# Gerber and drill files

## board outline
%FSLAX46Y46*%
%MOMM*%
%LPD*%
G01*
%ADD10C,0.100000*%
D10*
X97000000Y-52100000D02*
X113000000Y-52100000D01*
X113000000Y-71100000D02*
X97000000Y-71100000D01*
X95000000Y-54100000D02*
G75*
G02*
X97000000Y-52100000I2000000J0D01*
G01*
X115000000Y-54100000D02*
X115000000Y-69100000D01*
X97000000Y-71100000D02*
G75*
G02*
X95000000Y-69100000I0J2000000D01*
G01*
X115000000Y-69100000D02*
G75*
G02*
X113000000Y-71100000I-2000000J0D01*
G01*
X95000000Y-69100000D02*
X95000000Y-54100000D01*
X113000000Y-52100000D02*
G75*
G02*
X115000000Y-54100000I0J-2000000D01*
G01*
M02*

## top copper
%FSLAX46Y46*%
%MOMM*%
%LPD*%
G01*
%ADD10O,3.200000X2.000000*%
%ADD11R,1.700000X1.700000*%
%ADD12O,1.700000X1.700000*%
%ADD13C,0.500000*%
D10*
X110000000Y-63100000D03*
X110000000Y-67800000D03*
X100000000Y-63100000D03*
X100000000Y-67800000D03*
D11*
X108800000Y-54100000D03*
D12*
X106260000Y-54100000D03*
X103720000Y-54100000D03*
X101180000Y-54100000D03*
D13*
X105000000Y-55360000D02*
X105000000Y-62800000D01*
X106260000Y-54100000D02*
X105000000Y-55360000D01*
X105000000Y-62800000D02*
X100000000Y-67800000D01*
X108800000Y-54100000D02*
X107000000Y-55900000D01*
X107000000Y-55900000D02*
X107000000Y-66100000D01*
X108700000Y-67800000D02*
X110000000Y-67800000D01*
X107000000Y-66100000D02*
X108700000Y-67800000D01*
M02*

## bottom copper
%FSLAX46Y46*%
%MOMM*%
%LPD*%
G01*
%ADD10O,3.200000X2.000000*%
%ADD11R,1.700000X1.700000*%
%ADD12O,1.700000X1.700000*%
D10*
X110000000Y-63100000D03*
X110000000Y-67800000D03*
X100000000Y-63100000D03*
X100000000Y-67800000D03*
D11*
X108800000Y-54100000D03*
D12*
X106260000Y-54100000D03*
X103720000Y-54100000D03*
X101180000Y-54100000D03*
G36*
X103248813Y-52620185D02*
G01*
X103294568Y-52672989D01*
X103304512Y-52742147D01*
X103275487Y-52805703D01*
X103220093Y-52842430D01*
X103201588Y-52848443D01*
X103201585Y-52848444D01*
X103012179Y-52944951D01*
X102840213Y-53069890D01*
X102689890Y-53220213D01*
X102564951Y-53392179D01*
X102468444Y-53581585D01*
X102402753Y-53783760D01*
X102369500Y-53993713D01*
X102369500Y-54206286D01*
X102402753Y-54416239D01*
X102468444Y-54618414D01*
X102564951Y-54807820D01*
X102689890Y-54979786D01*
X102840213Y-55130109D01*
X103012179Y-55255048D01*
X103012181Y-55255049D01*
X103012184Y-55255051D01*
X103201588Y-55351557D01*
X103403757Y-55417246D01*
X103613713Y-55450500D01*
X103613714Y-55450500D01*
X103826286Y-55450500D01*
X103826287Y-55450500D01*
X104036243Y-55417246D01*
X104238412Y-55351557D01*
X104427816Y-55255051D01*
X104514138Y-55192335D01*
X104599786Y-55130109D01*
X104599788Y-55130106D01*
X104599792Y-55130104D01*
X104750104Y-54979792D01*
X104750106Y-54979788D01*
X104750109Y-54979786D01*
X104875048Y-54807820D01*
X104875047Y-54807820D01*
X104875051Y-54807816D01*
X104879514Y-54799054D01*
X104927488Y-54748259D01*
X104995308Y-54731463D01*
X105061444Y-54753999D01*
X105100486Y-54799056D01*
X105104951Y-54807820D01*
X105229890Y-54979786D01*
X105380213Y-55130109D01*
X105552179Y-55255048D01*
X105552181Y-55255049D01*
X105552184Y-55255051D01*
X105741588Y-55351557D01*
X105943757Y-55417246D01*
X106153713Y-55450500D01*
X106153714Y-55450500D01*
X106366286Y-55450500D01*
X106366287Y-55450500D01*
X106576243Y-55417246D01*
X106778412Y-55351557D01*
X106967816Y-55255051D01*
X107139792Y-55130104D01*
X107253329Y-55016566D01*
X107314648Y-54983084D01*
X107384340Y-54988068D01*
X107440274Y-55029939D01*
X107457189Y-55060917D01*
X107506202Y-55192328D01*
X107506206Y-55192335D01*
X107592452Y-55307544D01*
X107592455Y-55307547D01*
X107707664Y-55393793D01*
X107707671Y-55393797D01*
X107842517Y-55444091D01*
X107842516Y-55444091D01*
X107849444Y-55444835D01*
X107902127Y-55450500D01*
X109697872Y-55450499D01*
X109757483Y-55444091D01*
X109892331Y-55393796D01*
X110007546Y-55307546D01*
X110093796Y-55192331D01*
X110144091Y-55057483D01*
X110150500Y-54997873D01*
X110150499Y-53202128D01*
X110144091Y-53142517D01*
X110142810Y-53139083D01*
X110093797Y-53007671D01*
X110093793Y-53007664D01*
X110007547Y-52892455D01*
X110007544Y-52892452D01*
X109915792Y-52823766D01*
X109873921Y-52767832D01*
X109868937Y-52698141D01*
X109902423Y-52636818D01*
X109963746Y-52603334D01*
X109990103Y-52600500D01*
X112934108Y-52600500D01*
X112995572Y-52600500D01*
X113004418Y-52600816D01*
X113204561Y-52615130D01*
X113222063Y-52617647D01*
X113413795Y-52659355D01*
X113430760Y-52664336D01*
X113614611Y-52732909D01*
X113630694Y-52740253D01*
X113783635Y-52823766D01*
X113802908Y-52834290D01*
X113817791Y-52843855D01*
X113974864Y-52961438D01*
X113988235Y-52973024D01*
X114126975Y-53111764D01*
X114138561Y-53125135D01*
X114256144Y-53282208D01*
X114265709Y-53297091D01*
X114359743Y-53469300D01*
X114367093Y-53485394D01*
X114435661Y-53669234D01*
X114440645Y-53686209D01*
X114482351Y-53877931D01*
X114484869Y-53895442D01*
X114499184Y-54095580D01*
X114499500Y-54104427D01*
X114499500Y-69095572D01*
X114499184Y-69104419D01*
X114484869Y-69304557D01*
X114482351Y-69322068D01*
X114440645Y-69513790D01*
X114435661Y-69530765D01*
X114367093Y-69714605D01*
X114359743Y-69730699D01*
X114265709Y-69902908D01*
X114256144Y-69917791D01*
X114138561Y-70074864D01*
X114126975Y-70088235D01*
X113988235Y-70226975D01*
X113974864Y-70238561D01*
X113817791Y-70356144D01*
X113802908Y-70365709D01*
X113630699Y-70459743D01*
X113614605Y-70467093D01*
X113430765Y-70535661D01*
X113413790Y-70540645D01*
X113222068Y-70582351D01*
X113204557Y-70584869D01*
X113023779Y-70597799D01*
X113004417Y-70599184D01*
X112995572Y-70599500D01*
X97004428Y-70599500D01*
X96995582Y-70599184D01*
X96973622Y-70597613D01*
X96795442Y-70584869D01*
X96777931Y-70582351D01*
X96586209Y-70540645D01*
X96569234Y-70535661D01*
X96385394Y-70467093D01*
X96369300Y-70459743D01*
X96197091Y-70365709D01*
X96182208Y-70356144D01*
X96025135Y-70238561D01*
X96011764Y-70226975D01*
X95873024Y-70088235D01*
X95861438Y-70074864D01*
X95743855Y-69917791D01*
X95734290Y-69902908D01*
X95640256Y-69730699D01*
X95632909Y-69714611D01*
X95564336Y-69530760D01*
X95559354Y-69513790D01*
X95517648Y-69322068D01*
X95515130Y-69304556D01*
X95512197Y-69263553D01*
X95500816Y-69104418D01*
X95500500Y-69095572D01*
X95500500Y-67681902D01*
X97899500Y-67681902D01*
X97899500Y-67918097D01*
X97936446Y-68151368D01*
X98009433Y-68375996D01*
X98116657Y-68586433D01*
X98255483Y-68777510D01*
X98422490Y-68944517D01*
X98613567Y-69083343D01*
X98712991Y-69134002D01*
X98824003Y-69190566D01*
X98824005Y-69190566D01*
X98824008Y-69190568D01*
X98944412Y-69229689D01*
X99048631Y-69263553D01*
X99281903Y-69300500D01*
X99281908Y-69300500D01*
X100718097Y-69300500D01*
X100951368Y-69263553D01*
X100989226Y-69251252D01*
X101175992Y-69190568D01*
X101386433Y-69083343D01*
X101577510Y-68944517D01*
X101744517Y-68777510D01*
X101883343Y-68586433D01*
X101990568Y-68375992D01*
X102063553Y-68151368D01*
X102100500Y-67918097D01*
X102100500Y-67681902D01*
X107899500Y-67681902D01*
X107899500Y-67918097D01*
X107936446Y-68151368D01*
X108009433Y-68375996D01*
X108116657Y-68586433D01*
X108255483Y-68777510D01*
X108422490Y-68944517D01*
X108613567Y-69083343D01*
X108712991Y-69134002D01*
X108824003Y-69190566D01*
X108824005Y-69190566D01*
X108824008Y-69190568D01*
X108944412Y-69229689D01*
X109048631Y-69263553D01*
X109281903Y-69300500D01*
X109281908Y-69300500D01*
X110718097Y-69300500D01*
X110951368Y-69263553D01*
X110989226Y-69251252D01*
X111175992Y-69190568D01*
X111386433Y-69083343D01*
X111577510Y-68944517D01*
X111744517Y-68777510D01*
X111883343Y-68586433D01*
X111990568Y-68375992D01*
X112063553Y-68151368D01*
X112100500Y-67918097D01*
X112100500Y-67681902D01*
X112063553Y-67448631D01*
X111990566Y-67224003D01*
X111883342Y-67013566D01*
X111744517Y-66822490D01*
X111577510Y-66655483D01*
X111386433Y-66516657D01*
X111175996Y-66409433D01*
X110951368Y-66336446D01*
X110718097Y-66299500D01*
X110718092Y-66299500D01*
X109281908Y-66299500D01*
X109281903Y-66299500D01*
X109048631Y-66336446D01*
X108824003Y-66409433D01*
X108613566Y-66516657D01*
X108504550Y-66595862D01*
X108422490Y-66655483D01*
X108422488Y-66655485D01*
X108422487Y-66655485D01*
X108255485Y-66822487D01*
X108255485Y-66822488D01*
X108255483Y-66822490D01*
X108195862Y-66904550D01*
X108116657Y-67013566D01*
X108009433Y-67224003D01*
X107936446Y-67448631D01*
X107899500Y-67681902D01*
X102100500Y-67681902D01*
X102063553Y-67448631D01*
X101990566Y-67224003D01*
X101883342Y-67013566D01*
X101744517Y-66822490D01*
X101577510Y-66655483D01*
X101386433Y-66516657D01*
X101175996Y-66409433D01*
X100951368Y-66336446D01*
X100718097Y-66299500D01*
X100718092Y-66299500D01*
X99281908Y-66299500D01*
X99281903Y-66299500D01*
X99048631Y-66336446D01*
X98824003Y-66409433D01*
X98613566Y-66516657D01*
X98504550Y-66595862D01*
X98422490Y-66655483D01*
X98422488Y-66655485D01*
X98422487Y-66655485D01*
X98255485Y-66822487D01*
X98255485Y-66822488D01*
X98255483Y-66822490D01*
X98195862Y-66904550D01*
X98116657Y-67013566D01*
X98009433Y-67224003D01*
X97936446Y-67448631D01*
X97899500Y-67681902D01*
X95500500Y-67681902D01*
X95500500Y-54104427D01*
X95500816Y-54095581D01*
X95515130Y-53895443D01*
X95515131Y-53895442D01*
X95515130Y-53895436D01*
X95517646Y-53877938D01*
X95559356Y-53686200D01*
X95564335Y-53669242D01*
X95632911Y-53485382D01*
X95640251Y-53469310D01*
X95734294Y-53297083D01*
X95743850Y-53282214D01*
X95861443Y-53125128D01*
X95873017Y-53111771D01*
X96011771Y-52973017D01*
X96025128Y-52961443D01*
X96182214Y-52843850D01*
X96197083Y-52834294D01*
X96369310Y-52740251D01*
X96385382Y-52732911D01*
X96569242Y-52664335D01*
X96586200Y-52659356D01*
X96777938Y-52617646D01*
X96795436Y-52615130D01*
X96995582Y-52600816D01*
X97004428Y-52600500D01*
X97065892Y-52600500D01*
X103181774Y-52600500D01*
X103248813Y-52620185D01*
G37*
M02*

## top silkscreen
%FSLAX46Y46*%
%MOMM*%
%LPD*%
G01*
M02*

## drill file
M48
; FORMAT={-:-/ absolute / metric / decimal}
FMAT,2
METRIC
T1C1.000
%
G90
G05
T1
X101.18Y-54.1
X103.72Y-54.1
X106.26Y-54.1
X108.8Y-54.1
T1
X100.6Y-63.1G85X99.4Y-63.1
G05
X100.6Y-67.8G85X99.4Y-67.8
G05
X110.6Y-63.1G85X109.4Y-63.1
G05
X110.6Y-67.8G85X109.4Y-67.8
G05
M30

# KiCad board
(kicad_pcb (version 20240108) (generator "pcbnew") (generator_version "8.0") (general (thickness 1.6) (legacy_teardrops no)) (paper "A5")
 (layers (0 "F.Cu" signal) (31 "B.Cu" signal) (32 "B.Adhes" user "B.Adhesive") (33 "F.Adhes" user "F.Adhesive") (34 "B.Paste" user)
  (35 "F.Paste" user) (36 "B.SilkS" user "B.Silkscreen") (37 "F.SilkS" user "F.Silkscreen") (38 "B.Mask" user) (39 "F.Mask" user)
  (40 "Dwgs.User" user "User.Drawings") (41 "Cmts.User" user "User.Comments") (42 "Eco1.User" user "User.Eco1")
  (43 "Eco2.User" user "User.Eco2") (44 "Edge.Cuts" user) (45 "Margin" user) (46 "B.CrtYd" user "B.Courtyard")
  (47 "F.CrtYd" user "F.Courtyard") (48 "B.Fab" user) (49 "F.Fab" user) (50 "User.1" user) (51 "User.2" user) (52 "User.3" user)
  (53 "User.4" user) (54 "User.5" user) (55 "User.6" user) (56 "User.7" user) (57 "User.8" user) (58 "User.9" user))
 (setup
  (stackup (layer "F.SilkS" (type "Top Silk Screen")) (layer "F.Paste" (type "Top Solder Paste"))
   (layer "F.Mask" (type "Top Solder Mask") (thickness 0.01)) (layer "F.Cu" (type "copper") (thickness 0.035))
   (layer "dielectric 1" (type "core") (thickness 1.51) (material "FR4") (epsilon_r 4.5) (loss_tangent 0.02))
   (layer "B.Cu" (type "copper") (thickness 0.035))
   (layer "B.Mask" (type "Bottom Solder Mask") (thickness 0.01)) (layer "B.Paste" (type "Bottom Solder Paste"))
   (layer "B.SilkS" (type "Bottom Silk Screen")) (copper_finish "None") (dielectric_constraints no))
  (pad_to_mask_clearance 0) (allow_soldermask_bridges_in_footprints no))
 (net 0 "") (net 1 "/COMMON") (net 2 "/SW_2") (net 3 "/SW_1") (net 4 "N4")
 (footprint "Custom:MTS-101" (layer "F.Cu") (at 110 63.1 180)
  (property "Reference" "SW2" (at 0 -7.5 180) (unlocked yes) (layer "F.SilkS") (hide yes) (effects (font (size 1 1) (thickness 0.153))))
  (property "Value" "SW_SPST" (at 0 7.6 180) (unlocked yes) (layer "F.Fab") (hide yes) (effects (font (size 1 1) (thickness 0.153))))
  (pad "1" thru_hole oval (at 0 0 180) (size 3.2 2) (drill oval 2.2 1) (layers "*.Cu" "*.Mask") (remove_unused_layers no) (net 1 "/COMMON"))
  (pad "2" thru_hole oval (at 0 -4.7 180) (size 3.2 2) (drill oval 2.2 1) (layers "*.Cu" "*.Mask") (remove_unused_layers no) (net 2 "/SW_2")))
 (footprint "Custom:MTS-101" (layer "F.Cu") (at 100 63.1 180)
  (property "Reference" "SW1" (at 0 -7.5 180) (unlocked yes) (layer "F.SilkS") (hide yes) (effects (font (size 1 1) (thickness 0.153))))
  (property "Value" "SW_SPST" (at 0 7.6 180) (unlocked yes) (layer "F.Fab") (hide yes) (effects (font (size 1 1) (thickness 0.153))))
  (pad "1" thru_hole oval (at 0 0 180) (size 3.2 2) (drill oval 2.2 1) (layers "*.Cu" "*.Mask") (remove_unused_layers no) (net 1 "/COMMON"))
  (pad "2" thru_hole oval (at 0 -4.7 180) (size 3.2 2) (drill oval 2.2 1) (layers "*.Cu" "*.Mask") (remove_unused_layers no) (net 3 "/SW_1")))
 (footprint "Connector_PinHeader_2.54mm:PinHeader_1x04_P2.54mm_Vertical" (layer "B.Cu") (at 108.8 54.1 90)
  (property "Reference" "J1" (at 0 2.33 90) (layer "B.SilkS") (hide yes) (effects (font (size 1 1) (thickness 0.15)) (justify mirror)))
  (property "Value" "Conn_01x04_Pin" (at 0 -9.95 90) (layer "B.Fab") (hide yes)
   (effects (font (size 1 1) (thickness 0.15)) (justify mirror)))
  (pad "1" thru_hole rect (at 0 0 90) (size 1.7 1.7) (drill 1) (layers "*.Cu" "*.Mask") (remove_unused_layers no) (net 2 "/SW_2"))
  (pad "2" thru_hole oval (at 0 -2.54 90) (size 1.7 1.7) (drill 1) (layers "*.Cu" "*.Mask") (remove_unused_layers no) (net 3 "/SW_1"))
  (pad "3" thru_hole oval (at 0 -5.08 90) (size 1.7 1.7) (drill 1) (layers "*.Cu" "*.Mask") (remove_unused_layers no) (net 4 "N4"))
  (pad "4" thru_hole oval (at 0 -7.62 90) (size 1.7 1.7) (drill 1) (layers "*.Cu" "*.Mask") (remove_unused_layers no) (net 1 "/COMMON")))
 (gr_line (start 97 52.1) (end 113 52.1) (stroke (width 0.1) (type default)) (layer "Edge.Cuts"))
 (gr_line (start 113 71.1) (end 97 71.1) (stroke (width 0.1) (type default)) (layer "Edge.Cuts"))
 (gr_arc (start 95 54.1) (mid 95.585786 52.685786) (end 97 52.1) (stroke (width 0.1) (type default)) (layer "Edge.Cuts"))
 (gr_line (start 115 54.1) (end 115 69.1) (stroke (width 0.1) (type default)) (layer "Edge.Cuts"))
 (gr_arc (start 97 71.1) (mid 95.585786 70.514214) (end 95 69.1) (stroke (width 0.1) (type default)) (layer "Edge.Cuts"))
 (gr_arc (start 115 69.1) (mid 114.414214 70.514214) (end 113 71.1) (stroke (width 0.1) (type default)) (layer "Edge.Cuts"))
 (gr_line (start 95 69.1) (end 95 54.1) (stroke (width 0.1) (type default)) (layer "Edge.Cuts"))
 (gr_arc (start 113 52.1) (mid 114.414214 52.685786) (end 115 54.1) (stroke (width 0.1) (type default)) (layer "Edge.Cuts"))
 (segment (start 105 55.36) (end 105 62.8) (width 0.5) (layer "F.Cu") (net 3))
 (segment (start 106.26 54.1) (end 105 55.36) (width 0.5) (layer "F.Cu") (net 3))
 (segment (start 105 62.8) (end 100 67.8) (width 0.5) (layer "F.Cu") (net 3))
 (segment (start 108.8 54.1) (end 107 55.9) (width 0.5) (layer "F.Cu") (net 2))
 (segment (start 107 55.9) (end 107 66.1) (width 0.5) (layer "F.Cu") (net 2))
 (segment (start 108.7 67.8) (end 110 67.8) (width 0.5) (layer "F.Cu") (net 2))
 (segment (start 107 66.1) (end 108.7 67.8) (width 0.5) (layer "F.Cu") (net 2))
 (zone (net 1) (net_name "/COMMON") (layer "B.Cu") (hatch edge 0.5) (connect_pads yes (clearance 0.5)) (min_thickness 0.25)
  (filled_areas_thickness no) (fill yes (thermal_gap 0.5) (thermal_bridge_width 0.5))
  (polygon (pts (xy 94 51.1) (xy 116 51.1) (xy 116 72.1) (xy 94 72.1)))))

